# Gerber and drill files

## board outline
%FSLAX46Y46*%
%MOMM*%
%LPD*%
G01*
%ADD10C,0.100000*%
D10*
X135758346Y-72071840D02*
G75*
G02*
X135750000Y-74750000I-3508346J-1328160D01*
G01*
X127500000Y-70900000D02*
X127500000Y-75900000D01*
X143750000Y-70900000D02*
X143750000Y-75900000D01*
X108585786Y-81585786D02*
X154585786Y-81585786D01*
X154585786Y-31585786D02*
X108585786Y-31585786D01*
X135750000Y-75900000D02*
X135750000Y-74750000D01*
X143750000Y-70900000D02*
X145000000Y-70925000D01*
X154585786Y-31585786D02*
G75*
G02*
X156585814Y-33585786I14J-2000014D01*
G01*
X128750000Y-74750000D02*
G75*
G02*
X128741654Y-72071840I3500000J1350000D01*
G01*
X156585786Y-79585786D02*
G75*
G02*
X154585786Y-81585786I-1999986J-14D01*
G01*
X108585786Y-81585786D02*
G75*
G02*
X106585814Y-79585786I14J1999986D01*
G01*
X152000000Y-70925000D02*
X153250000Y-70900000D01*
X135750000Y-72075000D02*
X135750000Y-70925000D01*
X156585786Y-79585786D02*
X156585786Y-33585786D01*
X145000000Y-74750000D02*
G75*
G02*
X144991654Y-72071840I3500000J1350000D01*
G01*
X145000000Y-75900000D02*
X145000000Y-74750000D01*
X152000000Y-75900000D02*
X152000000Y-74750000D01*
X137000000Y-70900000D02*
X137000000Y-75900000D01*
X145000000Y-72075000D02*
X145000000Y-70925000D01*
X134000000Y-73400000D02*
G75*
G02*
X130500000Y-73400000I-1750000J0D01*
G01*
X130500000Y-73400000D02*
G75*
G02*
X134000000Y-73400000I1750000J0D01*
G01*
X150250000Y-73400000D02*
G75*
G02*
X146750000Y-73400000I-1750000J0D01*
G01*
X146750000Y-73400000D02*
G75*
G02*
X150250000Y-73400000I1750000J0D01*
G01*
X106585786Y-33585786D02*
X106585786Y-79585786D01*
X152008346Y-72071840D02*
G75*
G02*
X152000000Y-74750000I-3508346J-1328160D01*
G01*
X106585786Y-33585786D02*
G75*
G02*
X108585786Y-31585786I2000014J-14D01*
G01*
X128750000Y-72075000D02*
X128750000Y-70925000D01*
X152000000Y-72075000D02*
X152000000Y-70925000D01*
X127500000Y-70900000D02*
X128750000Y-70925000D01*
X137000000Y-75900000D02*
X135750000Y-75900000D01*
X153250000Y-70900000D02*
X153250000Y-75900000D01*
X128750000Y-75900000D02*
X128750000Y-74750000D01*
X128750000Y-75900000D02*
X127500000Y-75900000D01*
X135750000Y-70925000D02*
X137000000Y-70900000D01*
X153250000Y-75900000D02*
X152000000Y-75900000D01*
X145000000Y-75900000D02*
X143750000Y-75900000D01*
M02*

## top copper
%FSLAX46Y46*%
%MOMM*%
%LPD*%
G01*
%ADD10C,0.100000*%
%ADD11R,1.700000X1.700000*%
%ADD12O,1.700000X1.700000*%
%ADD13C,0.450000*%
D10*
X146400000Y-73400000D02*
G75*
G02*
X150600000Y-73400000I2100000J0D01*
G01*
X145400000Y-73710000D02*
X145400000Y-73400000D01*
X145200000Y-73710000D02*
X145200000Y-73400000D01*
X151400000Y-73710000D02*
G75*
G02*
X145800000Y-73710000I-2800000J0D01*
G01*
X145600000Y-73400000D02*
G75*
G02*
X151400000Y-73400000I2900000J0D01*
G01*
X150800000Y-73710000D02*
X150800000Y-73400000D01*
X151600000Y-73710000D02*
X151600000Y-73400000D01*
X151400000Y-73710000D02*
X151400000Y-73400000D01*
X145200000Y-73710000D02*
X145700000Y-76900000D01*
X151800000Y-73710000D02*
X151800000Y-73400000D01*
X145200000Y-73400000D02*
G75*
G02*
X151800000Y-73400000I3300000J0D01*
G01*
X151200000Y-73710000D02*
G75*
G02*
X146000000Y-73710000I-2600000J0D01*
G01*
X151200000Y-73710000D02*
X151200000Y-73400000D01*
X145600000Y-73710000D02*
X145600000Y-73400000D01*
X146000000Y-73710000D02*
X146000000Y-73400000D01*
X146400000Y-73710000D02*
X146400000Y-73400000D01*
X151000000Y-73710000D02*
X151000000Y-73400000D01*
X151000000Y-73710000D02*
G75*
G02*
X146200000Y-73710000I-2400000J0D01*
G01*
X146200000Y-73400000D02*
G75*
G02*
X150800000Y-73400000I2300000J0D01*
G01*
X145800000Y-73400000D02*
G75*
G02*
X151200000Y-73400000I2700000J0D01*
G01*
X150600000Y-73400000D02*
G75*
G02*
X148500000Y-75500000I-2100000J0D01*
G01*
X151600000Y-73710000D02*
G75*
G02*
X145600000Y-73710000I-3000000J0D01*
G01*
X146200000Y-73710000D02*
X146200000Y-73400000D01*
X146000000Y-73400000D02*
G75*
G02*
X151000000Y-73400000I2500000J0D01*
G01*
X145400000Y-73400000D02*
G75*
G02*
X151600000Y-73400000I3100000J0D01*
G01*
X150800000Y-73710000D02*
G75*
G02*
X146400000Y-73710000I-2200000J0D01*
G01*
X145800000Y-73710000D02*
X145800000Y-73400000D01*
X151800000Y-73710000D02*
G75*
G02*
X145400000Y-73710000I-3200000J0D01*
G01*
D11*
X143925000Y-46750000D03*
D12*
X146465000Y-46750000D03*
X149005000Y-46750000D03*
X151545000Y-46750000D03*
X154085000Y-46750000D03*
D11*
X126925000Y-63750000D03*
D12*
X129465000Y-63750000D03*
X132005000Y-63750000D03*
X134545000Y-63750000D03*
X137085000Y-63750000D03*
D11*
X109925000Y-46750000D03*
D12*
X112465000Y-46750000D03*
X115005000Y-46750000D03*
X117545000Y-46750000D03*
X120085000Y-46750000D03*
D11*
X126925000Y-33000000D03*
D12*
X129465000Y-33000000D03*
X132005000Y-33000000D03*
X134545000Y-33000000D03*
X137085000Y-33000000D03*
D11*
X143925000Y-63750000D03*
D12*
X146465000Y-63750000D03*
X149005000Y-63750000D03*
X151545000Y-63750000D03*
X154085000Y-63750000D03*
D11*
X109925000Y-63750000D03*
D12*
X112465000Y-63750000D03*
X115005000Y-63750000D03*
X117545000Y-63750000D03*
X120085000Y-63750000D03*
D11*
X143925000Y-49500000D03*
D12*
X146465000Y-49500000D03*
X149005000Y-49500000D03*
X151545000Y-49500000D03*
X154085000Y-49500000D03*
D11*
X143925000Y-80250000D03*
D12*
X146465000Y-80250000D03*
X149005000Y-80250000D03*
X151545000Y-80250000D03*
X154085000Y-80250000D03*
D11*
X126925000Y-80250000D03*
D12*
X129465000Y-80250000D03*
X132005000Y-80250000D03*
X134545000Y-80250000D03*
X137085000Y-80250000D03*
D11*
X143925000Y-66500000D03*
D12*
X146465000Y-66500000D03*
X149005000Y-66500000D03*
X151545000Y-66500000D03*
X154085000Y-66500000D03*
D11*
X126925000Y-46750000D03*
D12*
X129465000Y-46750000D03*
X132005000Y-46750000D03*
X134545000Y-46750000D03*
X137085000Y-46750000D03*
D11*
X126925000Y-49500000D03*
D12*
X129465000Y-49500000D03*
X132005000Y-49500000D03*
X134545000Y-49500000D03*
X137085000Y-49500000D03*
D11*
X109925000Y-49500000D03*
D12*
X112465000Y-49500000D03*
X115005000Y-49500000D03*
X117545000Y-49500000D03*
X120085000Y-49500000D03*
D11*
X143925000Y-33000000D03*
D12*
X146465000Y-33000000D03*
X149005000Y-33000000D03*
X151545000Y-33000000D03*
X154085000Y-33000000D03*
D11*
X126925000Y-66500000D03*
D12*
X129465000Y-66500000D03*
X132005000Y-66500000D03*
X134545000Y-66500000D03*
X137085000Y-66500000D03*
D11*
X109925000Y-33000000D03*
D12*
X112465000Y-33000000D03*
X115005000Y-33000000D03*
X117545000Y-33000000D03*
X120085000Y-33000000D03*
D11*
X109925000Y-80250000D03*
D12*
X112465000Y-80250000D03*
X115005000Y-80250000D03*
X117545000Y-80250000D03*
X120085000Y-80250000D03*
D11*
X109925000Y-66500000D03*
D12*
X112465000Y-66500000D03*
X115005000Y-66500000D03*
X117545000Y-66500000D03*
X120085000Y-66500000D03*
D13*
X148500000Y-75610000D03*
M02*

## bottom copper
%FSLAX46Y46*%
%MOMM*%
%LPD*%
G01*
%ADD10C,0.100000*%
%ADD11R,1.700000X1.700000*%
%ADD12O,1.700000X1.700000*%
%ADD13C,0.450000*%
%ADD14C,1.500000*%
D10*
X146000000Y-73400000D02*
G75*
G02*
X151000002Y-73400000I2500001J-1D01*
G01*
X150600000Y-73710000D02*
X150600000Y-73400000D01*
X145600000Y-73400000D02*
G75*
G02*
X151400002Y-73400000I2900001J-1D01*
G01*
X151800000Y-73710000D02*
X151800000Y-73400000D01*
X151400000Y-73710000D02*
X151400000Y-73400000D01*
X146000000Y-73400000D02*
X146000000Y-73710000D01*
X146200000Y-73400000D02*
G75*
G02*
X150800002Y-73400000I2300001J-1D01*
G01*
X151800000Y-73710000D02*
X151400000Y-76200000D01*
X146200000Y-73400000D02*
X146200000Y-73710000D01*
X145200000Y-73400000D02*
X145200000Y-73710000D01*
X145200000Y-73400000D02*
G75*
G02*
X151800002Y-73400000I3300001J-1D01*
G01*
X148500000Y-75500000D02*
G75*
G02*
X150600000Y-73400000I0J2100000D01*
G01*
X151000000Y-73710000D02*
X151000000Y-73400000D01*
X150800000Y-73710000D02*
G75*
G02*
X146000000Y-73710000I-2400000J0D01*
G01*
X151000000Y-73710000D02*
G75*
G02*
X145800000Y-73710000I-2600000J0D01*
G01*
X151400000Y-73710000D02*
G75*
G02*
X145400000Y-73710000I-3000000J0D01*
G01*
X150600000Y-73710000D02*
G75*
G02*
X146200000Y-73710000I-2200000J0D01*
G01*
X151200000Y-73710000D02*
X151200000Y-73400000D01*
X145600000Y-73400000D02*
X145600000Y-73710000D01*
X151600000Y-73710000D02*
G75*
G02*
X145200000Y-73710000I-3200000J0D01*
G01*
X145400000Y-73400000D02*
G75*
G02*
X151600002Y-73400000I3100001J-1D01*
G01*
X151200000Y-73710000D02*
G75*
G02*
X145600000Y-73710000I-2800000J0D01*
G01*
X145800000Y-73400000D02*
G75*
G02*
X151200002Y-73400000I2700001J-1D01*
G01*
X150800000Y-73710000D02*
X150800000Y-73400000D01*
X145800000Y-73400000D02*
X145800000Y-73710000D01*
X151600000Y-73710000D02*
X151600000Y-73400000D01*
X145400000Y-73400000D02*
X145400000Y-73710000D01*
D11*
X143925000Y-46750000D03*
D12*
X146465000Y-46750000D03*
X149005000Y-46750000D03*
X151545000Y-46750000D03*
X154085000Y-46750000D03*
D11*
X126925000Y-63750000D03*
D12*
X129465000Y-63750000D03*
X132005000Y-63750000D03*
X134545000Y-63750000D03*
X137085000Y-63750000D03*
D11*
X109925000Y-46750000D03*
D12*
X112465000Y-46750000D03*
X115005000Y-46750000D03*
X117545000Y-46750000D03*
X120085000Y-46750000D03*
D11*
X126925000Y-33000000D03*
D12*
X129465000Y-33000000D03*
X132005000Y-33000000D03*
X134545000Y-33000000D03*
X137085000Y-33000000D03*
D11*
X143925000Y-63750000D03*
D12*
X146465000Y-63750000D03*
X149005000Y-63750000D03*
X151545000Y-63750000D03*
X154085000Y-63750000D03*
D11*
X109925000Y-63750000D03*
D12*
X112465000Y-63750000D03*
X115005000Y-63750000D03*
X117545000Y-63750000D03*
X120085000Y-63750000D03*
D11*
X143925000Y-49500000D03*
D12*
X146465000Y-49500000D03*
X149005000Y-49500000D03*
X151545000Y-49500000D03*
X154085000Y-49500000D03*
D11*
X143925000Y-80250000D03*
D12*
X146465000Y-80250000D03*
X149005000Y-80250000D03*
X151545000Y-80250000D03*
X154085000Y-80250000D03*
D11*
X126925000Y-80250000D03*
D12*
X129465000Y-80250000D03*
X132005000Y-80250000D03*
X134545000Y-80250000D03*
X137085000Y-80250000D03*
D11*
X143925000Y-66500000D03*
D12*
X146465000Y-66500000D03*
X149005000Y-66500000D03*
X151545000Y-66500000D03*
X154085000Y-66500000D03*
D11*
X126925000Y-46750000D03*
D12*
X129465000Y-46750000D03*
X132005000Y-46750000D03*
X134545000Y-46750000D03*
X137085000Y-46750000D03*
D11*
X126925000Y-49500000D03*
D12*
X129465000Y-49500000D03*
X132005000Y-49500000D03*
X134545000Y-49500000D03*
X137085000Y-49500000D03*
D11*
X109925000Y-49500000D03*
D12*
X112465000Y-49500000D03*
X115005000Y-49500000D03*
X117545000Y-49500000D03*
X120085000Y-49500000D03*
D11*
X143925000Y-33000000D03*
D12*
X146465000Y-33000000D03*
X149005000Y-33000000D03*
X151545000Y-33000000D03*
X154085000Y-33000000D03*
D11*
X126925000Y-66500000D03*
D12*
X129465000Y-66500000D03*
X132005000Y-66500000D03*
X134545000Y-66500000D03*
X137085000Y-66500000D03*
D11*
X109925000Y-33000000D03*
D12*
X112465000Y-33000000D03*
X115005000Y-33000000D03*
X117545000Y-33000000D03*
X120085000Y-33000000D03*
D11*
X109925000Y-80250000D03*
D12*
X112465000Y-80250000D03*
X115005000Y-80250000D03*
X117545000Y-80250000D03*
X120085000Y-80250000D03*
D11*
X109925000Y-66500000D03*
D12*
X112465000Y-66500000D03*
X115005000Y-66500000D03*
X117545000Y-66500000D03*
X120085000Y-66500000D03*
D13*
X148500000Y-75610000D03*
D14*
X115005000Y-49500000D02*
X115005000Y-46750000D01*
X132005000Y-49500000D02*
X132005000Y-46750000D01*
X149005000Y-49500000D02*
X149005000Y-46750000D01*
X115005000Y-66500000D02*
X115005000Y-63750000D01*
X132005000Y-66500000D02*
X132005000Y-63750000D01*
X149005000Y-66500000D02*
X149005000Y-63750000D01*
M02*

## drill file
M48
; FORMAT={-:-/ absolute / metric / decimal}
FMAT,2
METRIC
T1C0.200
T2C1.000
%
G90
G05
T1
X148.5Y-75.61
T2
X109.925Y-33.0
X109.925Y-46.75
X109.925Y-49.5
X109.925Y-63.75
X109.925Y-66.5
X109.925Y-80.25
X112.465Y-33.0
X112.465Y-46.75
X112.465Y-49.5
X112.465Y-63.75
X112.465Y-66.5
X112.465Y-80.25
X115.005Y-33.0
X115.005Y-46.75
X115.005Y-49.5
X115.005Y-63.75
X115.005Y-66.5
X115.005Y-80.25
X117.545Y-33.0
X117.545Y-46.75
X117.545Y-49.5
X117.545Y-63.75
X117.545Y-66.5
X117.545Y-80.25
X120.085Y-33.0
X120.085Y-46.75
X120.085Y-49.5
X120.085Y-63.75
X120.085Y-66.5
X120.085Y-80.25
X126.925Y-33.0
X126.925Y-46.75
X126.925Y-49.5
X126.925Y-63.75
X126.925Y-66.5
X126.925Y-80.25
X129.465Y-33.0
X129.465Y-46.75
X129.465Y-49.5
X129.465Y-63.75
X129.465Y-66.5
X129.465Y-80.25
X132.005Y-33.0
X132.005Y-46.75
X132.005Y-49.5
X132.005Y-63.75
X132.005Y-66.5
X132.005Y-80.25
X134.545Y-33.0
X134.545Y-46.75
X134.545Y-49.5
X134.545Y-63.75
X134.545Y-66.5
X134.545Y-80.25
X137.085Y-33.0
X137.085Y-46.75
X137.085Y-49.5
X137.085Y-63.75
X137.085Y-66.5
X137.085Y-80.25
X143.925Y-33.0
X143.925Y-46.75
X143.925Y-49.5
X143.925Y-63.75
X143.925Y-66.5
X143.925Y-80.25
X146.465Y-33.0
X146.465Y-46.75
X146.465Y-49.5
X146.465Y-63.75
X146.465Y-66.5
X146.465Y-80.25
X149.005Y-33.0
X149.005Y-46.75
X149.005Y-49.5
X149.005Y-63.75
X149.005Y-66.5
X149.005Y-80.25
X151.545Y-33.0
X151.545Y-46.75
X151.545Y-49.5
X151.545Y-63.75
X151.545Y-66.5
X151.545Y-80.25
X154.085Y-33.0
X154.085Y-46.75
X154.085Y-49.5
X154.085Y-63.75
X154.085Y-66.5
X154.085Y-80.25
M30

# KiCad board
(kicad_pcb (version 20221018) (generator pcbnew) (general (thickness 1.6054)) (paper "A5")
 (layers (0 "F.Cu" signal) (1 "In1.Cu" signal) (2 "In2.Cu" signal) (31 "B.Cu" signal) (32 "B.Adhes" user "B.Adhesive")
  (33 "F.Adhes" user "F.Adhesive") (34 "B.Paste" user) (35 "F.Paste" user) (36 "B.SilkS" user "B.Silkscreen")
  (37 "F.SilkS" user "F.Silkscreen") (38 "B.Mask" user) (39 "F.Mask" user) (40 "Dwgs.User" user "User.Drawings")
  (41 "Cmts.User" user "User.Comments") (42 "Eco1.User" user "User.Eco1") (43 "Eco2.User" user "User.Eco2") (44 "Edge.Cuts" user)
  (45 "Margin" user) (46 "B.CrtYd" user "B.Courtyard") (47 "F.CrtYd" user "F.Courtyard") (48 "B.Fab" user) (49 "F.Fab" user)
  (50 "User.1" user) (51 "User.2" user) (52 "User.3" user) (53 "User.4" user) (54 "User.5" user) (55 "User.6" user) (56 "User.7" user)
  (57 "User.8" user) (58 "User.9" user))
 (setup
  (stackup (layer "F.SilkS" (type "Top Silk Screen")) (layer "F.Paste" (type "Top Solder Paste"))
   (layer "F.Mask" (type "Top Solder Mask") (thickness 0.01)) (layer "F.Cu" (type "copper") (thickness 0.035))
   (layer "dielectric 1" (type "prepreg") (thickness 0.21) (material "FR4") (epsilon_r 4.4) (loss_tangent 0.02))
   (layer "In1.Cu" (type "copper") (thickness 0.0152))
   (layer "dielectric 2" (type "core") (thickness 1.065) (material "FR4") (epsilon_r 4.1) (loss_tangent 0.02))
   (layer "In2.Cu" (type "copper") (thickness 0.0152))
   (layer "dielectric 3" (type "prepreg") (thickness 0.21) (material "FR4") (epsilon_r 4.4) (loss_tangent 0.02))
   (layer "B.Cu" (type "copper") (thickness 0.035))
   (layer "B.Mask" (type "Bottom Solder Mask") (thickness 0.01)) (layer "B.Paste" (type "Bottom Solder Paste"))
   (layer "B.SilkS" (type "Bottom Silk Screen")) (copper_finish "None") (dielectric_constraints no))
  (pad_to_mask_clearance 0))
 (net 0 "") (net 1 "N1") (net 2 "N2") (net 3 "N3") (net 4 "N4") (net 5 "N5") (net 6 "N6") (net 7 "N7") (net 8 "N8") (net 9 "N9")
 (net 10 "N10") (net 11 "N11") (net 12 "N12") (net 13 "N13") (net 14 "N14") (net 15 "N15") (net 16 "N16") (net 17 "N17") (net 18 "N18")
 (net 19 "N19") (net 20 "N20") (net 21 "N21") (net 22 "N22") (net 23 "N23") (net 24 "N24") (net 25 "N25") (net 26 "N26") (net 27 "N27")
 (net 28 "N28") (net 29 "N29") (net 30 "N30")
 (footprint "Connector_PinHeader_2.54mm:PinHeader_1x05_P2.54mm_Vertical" (layer "F.Cu") (at 143.925 46.75 90)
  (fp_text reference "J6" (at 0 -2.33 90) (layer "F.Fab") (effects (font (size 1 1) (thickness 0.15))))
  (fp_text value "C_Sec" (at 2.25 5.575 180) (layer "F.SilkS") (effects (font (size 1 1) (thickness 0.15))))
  (pad "1" thru_hole rect (at 0 0 90) (size 1.7 1.7) (drill 1) (layers "*.Cu" "*.Mask") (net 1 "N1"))
  (pad "2" thru_hole oval (at 0 2.54 90) (size 1.7 1.7) (drill 1) (layers "*.Cu" "*.Mask") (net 1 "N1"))
  (pad "3" thru_hole oval (at 0 5.08 90) (size 1.7 1.7) (drill 1) (layers "*.Cu" "*.Mask") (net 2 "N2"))
  (pad "4" thru_hole oval (at 0 7.62 90) (size 1.7 1.7) (drill 1) (layers "*.Cu" "*.Mask") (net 1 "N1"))
  (pad "5" thru_hole oval (at 0 10.16 90) (size 1.7 1.7) (drill 1) (layers "*.Cu" "*.Mask") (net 1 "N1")))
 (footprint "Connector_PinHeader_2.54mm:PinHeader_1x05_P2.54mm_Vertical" (layer "F.Cu") (at 126.925 63.75 90)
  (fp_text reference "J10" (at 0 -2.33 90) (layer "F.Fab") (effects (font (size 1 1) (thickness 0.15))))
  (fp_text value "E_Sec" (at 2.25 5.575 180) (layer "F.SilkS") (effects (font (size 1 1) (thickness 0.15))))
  (pad "1" thru_hole rect (at 0 0 90) (size 1.7 1.7) (drill 1) (layers "*.Cu" "*.Mask") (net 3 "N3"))
  (pad "2" thru_hole oval (at 0 2.54 90) (size 1.7 1.7) (drill 1) (layers "*.Cu" "*.Mask") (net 3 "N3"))
  (pad "3" thru_hole oval (at 0 5.08 90) (size 1.7 1.7) (drill 1) (layers "*.Cu" "*.Mask") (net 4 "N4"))
  (pad "4" thru_hole oval (at 0 7.62 90) (size 1.7 1.7) (drill 1) (layers "*.Cu" "*.Mask") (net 3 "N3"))
  (pad "5" thru_hole oval (at 0 10.16 90) (size 1.7 1.7) (drill 1) (layers "*.Cu" "*.Mask") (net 3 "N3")))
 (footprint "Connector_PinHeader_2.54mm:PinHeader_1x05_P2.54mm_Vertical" (layer "F.Cu") (at 109.925 46.75 90)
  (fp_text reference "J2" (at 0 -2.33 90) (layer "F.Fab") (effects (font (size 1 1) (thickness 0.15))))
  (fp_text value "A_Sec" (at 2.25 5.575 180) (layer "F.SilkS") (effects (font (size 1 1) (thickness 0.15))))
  (pad "1" thru_hole rect (at 0 0 90) (size 1.7 1.7) (drill 1) (layers "*.Cu" "*.Mask") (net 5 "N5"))
  (pad "2" thru_hole oval (at 0 2.54 90) (size 1.7 1.7) (drill 1) (layers "*.Cu" "*.Mask") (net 5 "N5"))
  (pad "3" thru_hole oval (at 0 5.08 90) (size 1.7 1.7) (drill 1) (layers "*.Cu" "*.Mask") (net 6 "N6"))
  (pad "4" thru_hole oval (at 0 7.62 90) (size 1.7 1.7) (drill 1) (layers "*.Cu" "*.Mask") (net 5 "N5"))
  (pad "5" thru_hole oval (at 0 10.16 90) (size 1.7 1.7) (drill 1) (layers "*.Cu" "*.Mask") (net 5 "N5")))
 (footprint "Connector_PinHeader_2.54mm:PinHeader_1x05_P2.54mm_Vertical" (layer "F.Cu") (at 126.925 33 90)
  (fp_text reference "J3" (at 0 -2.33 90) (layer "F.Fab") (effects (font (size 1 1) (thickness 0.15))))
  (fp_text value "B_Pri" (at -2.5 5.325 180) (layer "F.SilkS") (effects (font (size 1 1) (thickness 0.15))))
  (pad "1" thru_hole rect (at 0 0 90) (size 1.7 1.7) (drill 1) (layers "*.Cu" "*.Mask") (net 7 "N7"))
  (pad "2" thru_hole oval (at 0 2.54 90) (size 1.7 1.7) (drill 1) (layers "*.Cu" "*.Mask") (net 7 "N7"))
  (pad "3" thru_hole oval (at 0 5.08 90) (size 1.7 1.7) (drill 1) (layers "*.Cu" "*.Mask") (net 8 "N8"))
  (pad "4" thru_hole oval (at 0 7.62 90) (size 1.7 1.7) (drill 1) (layers "*.Cu" "*.Mask") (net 7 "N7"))
  (pad "5" thru_hole oval (at 0 10.16 90) (size 1.7 1.7) (drill 1) (layers "*.Cu" "*.Mask") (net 7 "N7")))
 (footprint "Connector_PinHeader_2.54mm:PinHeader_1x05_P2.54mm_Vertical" (layer "F.Cu") (at 143.925 63.75 90)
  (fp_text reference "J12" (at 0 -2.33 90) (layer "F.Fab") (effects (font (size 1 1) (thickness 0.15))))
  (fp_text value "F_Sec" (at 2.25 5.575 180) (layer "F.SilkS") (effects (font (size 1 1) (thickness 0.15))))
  (pad "1" thru_hole rect (at 0 0 90) (size 1.7 1.7) (drill 1) (layers "*.Cu" "*.Mask") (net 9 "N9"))
  (pad "2" thru_hole oval (at 0 2.54 90) (size 1.7 1.7) (drill 1) (layers "*.Cu" "*.Mask") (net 9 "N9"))
  (pad "3" thru_hole oval (at 0 5.08 90) (size 1.7 1.7) (drill 1) (layers "*.Cu" "*.Mask") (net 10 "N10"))
  (pad "4" thru_hole oval (at 0 7.62 90) (size 1.7 1.7) (drill 1) (layers "*.Cu" "*.Mask") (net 9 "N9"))
  (pad "5" thru_hole oval (at 0 10.16 90) (size 1.7 1.7) (drill 1) (layers "*.Cu" "*.Mask") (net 9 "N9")))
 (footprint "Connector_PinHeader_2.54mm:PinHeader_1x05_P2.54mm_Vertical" (layer "F.Cu") (at 109.925 63.75 90)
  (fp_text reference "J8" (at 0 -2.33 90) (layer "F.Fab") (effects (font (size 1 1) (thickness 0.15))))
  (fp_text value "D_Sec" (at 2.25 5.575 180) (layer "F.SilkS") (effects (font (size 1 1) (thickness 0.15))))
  (pad "1" thru_hole rect (at 0 0 90) (size 1.7 1.7) (drill 1) (layers "*.Cu" "*.Mask") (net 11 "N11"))
  (pad "2" thru_hole oval (at 0 2.54 90) (size 1.7 1.7) (drill 1) (layers "*.Cu" "*.Mask") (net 11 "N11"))
  (pad "3" thru_hole oval (at 0 5.08 90) (size 1.7 1.7) (drill 1) (layers "*.Cu" "*.Mask") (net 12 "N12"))
  (pad "4" thru_hole oval (at 0 7.62 90) (size 1.7 1.7) (drill 1) (layers "*.Cu" "*.Mask") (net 11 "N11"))
  (pad "5" thru_hole oval (at 0 10.16 90) (size 1.7 1.7) (drill 1) (layers "*.Cu" "*.Mask") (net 11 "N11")))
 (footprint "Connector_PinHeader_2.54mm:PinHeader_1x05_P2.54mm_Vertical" (layer "F.Cu") (at 143.925 49.5 90)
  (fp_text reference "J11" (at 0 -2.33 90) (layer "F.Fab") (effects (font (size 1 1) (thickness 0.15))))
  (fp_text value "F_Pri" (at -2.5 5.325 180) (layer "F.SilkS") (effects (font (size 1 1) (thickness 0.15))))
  (pad "1" thru_hole rect (at 0 0 90) (size 1.7 1.7) (drill 1) (layers "*.Cu" "*.Mask") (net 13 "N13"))
  (pad "2" thru_hole oval (at 0 2.54 90) (size 1.7 1.7) (drill 1) (layers "*.Cu" "*.Mask") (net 13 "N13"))
  (pad "3" thru_hole oval (at 0 5.08 90) (size 1.7 1.7) (drill 1) (layers "*.Cu" "*.Mask") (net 2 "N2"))
  (pad "4" thru_hole oval (at 0 7.62 90) (size 1.7 1.7) (drill 1) (layers "*.Cu" "*.Mask") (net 13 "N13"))
  (pad "5" thru_hole oval (at 0 10.16 90) (size 1.7 1.7) (drill 1) (layers "*.Cu" "*.Mask") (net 13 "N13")))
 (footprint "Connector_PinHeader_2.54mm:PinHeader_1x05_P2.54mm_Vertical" (layer "F.Cu") (at 143.925 80.25 90)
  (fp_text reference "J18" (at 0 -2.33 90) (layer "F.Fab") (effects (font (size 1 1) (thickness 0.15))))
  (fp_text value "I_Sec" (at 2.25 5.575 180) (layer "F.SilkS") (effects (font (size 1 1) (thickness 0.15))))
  (pad "1" thru_hole rect (at 0 0 90) (size 1.7 1.7) (drill 1) (layers "*.Cu" "*.Mask") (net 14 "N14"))
  (pad "2" thru_hole oval (at 0 2.54 90) (size 1.7 1.7) (drill 1) (layers "*.Cu" "*.Mask") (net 14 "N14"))
  (pad "3" thru_hole oval (at 0 5.08 90) (size 1.7 1.7) (drill 1) (layers "*.Cu" "*.Mask") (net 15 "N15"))
  (pad "4" thru_hole oval (at 0 7.62 90) (size 1.7 1.7) (drill 1) (layers "*.Cu" "*.Mask") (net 14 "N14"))
  (pad "5" thru_hole oval (at 0 10.16 90) (size 1.7 1.7) (drill 1) (layers "*.Cu" "*.Mask") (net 14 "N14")))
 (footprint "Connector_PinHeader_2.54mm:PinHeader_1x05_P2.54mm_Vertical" (layer "F.Cu") (at 126.925 80.25 90)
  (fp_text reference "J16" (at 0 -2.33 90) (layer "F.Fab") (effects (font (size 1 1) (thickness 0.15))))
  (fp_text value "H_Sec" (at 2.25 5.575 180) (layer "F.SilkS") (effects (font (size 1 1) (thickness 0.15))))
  (pad "1" thru_hole rect (at 0 0 90) (size 1.7 1.7) (drill 1) (layers "*.Cu" "*.Mask") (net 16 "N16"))
  (pad "2" thru_hole oval (at 0 2.54 90) (size 1.7 1.7) (drill 1) (layers "*.Cu" "*.Mask") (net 16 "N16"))
  (pad "3" thru_hole oval (at 0 5.08 90) (size 1.7 1.7) (drill 1) (layers "*.Cu" "*.Mask") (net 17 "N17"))
  (pad "4" thru_hole oval (at 0 7.62 90) (size 1.7 1.7) (drill 1) (layers "*.Cu" "*.Mask") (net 16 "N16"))
  (pad "5" thru_hole oval (at 0 10.16 90) (size 1.7 1.7) (drill 1) (layers "*.Cu" "*.Mask") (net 16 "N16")))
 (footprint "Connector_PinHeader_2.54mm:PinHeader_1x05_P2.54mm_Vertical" (layer "F.Cu") (at 143.925 66.5 90)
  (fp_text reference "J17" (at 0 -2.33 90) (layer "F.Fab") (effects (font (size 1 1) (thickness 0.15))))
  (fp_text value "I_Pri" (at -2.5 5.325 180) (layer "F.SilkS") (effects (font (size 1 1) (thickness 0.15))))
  (pad "1" thru_hole rect (at 0 0 90) (size 1.7 1.7) (drill 1) (layers "*.Cu" "*.Mask") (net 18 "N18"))
  (pad "2" thru_hole oval (at 0 2.54 90) (size 1.7 1.7) (drill 1) (layers "*.Cu" "*.Mask") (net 18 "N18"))
  (pad "3" thru_hole oval (at 0 5.08 90) (size 1.7 1.7) (drill 1) (layers "*.Cu" "*.Mask") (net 10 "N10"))
  (pad "4" thru_hole oval (at 0 7.62 90) (size 1.7 1.7) (drill 1) (layers "*.Cu" "*.Mask") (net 18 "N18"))
  (pad "5" thru_hole oval (at 0 10.16 90) (size 1.7 1.7) (drill 1) (layers "*.Cu" "*.Mask") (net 18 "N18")))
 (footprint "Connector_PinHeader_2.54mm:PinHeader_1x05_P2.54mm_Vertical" (layer "F.Cu") (at 126.925 46.75 90)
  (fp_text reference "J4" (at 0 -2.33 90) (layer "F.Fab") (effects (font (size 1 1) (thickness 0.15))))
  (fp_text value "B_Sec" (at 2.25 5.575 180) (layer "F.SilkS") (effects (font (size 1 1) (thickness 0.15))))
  (pad "1" thru_hole rect (at 0 0 90) (size 1.7 1.7) (drill 1) (layers "*.Cu" "*.Mask") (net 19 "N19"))
  (pad "2" thru_hole oval (at 0 2.54 90) (size 1.7 1.7) (drill 1) (layers "*.Cu" "*.Mask") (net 19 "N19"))
  (pad "3" thru_hole oval (at 0 5.08 90) (size 1.7 1.7) (drill 1) (layers "*.Cu" "*.Mask") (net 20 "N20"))
  (pad "4" thru_hole oval (at 0 7.62 90) (size 1.7 1.7) (drill 1) (layers "*.Cu" "*.Mask") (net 19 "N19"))
  (pad "5" thru_hole oval (at 0 10.16 90) (size 1.7 1.7) (drill 1) (layers "*.Cu" "*.Mask") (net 19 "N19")))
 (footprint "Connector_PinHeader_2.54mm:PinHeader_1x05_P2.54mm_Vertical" (layer "F.Cu") (at 126.925 49.5 90)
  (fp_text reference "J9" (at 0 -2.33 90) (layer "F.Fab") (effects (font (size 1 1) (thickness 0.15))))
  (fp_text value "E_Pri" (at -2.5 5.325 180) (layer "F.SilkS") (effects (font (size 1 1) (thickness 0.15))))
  (pad "1" thru_hole rect (at 0 0 90) (size 1.7 1.7) (drill 1) (layers "*.Cu" "*.Mask") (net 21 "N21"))
  (pad "2" thru_hole oval (at 0 2.54 90) (size 1.7 1.7) (drill 1) (layers "*.Cu" "*.Mask") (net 21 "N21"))
  (pad "3" thru_hole oval (at 0 5.08 90) (size 1.7 1.7) (drill 1) (layers "*.Cu" "*.Mask") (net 20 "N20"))
  (pad "4" thru_hole oval (at 0 7.62 90) (size 1.7 1.7) (drill 1) (layers "*.Cu" "*.Mask") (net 21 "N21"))
  (pad "5" thru_hole oval (at 0 10.16 90) (size 1.7 1.7) (drill 1) (layers "*.Cu" "*.Mask") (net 21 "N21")))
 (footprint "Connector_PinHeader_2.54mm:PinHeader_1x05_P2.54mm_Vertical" (layer "F.Cu") (at 109.925 49.5 90)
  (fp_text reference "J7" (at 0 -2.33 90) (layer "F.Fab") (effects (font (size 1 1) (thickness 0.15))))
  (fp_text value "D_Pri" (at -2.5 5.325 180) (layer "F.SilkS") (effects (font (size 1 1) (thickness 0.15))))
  (pad "1" thru_hole rect (at 0 0 90) (size 1.7 1.7) (drill 1) (layers "*.Cu" "*.Mask") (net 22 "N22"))
  (pad "2" thru_hole oval (at 0 2.54 90) (size 1.7 1.7) (drill 1) (layers "*.Cu" "*.Mask") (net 22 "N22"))
  (pad "3" thru_hole oval (at 0 5.08 90) (size 1.7 1.7) (drill 1) (layers "*.Cu" "*.Mask") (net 6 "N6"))
  (pad "4" thru_hole oval (at 0 7.62 90) (size 1.7 1.7) (drill 1) (layers "*.Cu" "*.Mask") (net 22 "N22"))
  (pad "5" thru_hole oval (at 0 10.16 90) (size 1.7 1.7) (drill 1) (layers "*.Cu" "*.Mask") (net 22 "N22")))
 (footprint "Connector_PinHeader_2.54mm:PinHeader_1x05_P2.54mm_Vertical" (layer "F.Cu") (at 143.925 33 90)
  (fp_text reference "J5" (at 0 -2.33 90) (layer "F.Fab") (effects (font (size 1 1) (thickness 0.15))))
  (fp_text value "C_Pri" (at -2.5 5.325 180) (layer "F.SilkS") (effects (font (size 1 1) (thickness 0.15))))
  (pad "1" thru_hole rect (at 0 0 90) (size 1.7 1.7) (drill 1) (layers "*.Cu" "*.Mask") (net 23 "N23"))
  (pad "2" thru_hole oval (at 0 2.54 90) (size 1.7 1.7) (drill 1) (layers "*.Cu" "*.Mask") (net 23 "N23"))
  (pad "3" thru_hole oval (at 0 5.08 90) (size 1.7 1.7) (drill 1) (layers "*.Cu" "*.Mask") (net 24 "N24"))
  (pad "4" thru_hole oval (at 0 7.62 90) (size 1.7 1.7) (drill 1) (layers "*.Cu" "*.Mask") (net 23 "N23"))
  (pad "5" thru_hole oval (at 0 10.16 90) (size 1.7 1.7) (drill 1) (layers "*.Cu" "*.Mask") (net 23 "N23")))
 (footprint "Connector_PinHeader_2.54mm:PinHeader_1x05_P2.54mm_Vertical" (layer "F.Cu") (at 126.925 66.5 90)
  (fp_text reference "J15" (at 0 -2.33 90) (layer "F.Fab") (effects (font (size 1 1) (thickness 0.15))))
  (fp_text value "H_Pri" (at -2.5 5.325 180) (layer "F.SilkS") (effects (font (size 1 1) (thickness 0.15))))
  (pad "1" thru_hole rect (at 0 0 90) (size 1.7 1.7) (drill 1) (layers "*.Cu" "*.Mask") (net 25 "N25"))
  (pad "2" thru_hole oval (at 0 2.54 90) (size 1.7 1.7) (drill 1) (layers "*.Cu" "*.Mask") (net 25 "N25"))
  (pad "3" thru_hole oval (at 0 5.08 90) (size 1.7 1.7) (drill 1) (layers "*.Cu" "*.Mask") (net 4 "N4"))
  (pad "4" thru_hole oval (at 0 7.62 90) (size 1.7 1.7) (drill 1) (layers "*.Cu" "*.Mask") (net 25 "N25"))
  (pad "5" thru_hole oval (at 0 10.16 90) (size 1.7 1.7) (drill 1) (layers "*.Cu" "*.Mask") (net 25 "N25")))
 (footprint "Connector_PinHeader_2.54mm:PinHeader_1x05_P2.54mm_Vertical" (layer "F.Cu") (at 109.925 33 90)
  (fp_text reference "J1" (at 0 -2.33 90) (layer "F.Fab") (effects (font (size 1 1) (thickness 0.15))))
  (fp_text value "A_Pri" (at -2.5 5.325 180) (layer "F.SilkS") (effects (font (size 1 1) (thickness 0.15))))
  (pad "1" thru_hole rect (at 0 0 90) (size 1.7 1.7) (drill 1) (layers "*.Cu" "*.Mask") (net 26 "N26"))
  (pad "2" thru_hole oval (at 0 2.54 90) (size 1.7 1.7) (drill 1) (layers "*.Cu" "*.Mask") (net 26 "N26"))
  (pad "3" thru_hole oval (at 0 5.08 90) (size 1.7 1.7) (drill 1) (layers "*.Cu" "*.Mask") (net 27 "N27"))
  (pad "4" thru_hole oval (at 0 7.62 90) (size 1.7 1.7) (drill 1) (layers "*.Cu" "*.Mask") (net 26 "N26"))
  (pad "5" thru_hole oval (at 0 10.16 90) (size 1.7 1.7) (drill 1) (layers "*.Cu" "*.Mask") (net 26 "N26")))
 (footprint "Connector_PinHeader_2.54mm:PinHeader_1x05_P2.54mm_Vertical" (layer "F.Cu") (at 109.925 80.25 90)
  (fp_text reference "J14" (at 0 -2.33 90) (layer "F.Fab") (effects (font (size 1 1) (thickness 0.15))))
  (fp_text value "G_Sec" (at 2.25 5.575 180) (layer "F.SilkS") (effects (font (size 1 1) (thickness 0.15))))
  (pad "1" thru_hole rect (at 0 0 90) (size 1.7 1.7) (drill 1) (layers "*.Cu" "*.Mask") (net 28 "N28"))
  (pad "2" thru_hole oval (at 0 2.54 90) (size 1.7 1.7) (drill 1) (layers "*.Cu" "*.Mask") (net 28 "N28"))
  (pad "3" thru_hole oval (at 0 5.08 90) (size 1.7 1.7) (drill 1) (layers "*.Cu" "*.Mask") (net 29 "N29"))
  (pad "4" thru_hole oval (at 0 7.62 90) (size 1.7 1.7) (drill 1) (layers "*.Cu" "*.Mask") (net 28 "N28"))
  (pad "5" thru_hole oval (at 0 10.16 90) (size 1.7 1.7) (drill 1) (layers "*.Cu" "*.Mask") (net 28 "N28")))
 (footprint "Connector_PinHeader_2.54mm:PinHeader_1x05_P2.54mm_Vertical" (layer "F.Cu") (at 109.925 66.5 90)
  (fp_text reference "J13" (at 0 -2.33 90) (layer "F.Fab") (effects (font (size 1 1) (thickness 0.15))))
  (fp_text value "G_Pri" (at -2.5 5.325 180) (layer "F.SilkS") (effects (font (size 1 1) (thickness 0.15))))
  (pad "1" thru_hole rect (at 0 0 90) (size 1.7 1.7) (drill 1) (layers "*.Cu" "*.Mask") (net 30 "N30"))
  (pad "2" thru_hole oval (at 0 2.54 90) (size 1.7 1.7) (drill 1) (layers "*.Cu" "*.Mask") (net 30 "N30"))
  (pad "3" thru_hole oval (at 0 5.08 90) (size 1.7 1.7) (drill 1) (layers "*.Cu" "*.Mask") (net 12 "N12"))
  (pad "4" thru_hole oval (at 0 7.62 90) (size 1.7 1.7) (drill 1) (layers "*.Cu" "*.Mask") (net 30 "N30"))
  (pad "5" thru_hole oval (at 0 10.16 90) (size 1.7 1.7) (drill 1) (layers "*.Cu" "*.Mask") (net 30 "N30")))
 (gr_arc (start 146.4 73.4) (mid 148.5 71.3) (end 150.6 73.4) (stroke (width 0.1) (type default)) (layer "F.Cu"))
 (gr_line (start 145.4 73.71) (end 145.4 73.4) (stroke (width 0.1) (type default)) (layer "F.Cu"))
 (gr_line (start 145.2 73.71) (end 145.2 73.4) (stroke (width 0.1) (type default)) (layer "F.Cu"))
 (gr_arc (start 151.4 73.71) (mid 148.6 76.51) (end 145.8 73.71) (stroke (width 0.1) (type default)) (layer "F.Cu"))
 (gr_arc (start 145.6 73.4) (mid 148.5 70.5) (end 151.4 73.4) (stroke (width 0.1) (type default)) (layer "F.Cu"))
 (gr_line (start 150.8 73.71) (end 150.8 73.4) (stroke (width 0.1) (type default)) (layer "F.Cu"))
 (gr_line (start 151.6 73.71) (end 151.6 73.4) (stroke (width 0.1) (type default)) (layer "F.Cu"))
 (gr_line (start 151.4 73.71) (end 151.4 73.4) (stroke (width 0.1) (type default)) (layer "F.Cu"))
 (gr_line (start 145.2 73.71) (end 145.7 76.9) (stroke (width 0.1) (type default)) (layer "F.Cu"))
 (gr_line (start 151.8 73.71) (end 151.8 73.4) (stroke (width 0.1) (type default)) (layer "F.Cu"))
 (gr_arc (start 145.2 73.4) (mid 148.5 70.1) (end 151.8 73.4) (stroke (width 0.1) (type default)) (layer "F.Cu"))
 (gr_arc (start 151.2 73.71) (mid 148.6 76.31) (end 146 73.71) (stroke (width 0.1) (type default)) (layer "F.Cu"))
 (gr_line (start 151.2 73.71) (end 151.2 73.4) (stroke (width 0.1) (type default)) (layer "F.Cu"))
 (gr_line (start 145.6 73.71) (end 145.6 73.4) (stroke (width 0.1) (type default)) (layer "F.Cu"))
 (gr_line (start 146 73.71) (end 146 73.4) (stroke (width 0.1) (type default)) (layer "F.Cu"))
 (gr_line (start 146.4 73.71) (end 146.4 73.4) (stroke (width 0.1) (type default)) (layer "F.Cu"))
 (gr_line (start 151 73.71) (end 151 73.4) (stroke (width 0.1) (type default)) (layer "F.Cu"))
 (gr_arc (start 151 73.71) (mid 148.6 76.11) (end 146.2 73.71) (stroke (width 0.1) (type default)) (layer "F.Cu"))
 (gr_arc (start 146.2 73.4) (mid 148.5 71.1) (end 150.8 73.4) (stroke (width 0.1) (type default)) (layer "F.Cu"))
 (gr_arc (start 145.8 73.4) (mid 148.5 70.7) (end 151.2 73.4) (stroke (width 0.1) (type default)) (layer "F.Cu"))
 (gr_arc (start 150.6 73.4) (mid 149.984924 74.884924) (end 148.5 75.5) (stroke (width 0.1) (type default)) (layer "F.Cu"))
 (gr_arc (start 151.6 73.71) (mid 148.6 76.71) (end 145.6 73.71) (stroke (width 0.1) (type default)) (layer "F.Cu"))
 (gr_line (start 146.2 73.71) (end 146.2 73.4) (stroke (width 0.1) (type default)) (layer "F.Cu"))
 (gr_arc (start 146 73.4) (mid 148.5 70.9) (end 151 73.4) (stroke (width 0.1) (type default)) (layer "F.Cu"))
 (gr_arc (start 145.4 73.4) (mid 148.5 70.3) (end 151.6 73.4) (stroke (width 0.1) (type default)) (layer "F.Cu"))
 (gr_arc (start 150.8 73.71) (mid 148.6 75.91) (end 146.4 73.71) (stroke (width 0.1) (type default)) (layer "F.Cu"))
 (gr_line (start 145.8 73.71) (end 145.8 73.4) (stroke (width 0.1) (type default)) (layer "F.Cu"))
 (gr_arc (start 151.8 73.71) (mid 148.6 76.91) (end 145.4 73.71) (stroke (width 0.1) (type default)) (layer "F.Cu"))
 (gr_arc (start 146 73.4) (mid 148.500001 70.9) (end 151.000002 73.4) (stroke (width 0.1) (type default)) (layer "B.Cu"))
 (gr_line (start 150.6 73.71) (end 150.6 73.4) (stroke (width 0.1) (type default)) (layer "B.Cu"))
 (gr_arc (start 145.6 73.4) (mid 148.500001 70.5) (end 151.400002 73.4) (stroke (width 0.1) (type default)) (layer "B.Cu"))
 (gr_line (start 151.8 73.71) (end 151.8 73.4) (stroke (width 0.1) (type default)) (layer "B.Cu"))
 (gr_line (start 151.4 73.71) (end 151.4 73.4) (stroke (width 0.1) (type default)) (layer "B.Cu"))
 (gr_line (start 146 73.4) (end 146 73.71) (stroke (width 0.1) (type default)) (layer "B.Cu"))
 (gr_arc (start 146.2 73.4) (mid 148.500001 71.1) (end 150.800002 73.4) (stroke (width 0.1) (type default)) (layer "B.Cu"))
 (gr_line (start 151.8 73.71) (end 151.4 76.2) (stroke (width 0.1) (type default)) (layer "B.Cu"))
 (gr_line (start 146.2 73.4) (end 146.2 73.71) (stroke (width 0.1) (type default)) (layer "B.Cu"))
 (gr_line (start 145.2 73.4) (end 145.2 73.71) (stroke (width 0.1) (type default)) (layer "B.Cu"))
 (gr_arc (start 145.2 73.4) (mid 148.500001 70.1) (end 151.800002 73.4) (stroke (width 0.1) (type default)) (layer "B.Cu"))
 (gr_arc (start 148.5 75.5) (mid 147.015077 71.915077) (end 150.6 73.4) (stroke (width 0.1) (type default)) (layer "B.Cu"))
 (gr_line (start 151 73.71) (end 151 73.4) (stroke (width 0.1) (type default)) (layer "B.Cu"))
 (gr_arc (start 150.8 73.71) (mid 148.4 76.11) (end 146 73.71) (stroke (width 0.1) (type default)) (layer "B.Cu"))
 (gr_arc (start 151 73.71) (mid 148.4 76.31) (end 145.8 73.71) (stroke (width 0.1) (type default)) (layer "B.Cu"))
 (gr_arc (start 151.4 73.71) (mid 148.4 76.71) (end 145.4 73.71) (stroke (width 0.1) (type default)) (layer "B.Cu"))
 (gr_arc (start 150.6 73.71) (mid 148.4 75.91) (end 146.2 73.71) (stroke (width 0.1) (type default)) (layer "B.Cu"))
 (gr_line (start 151.2 73.71) (end 151.2 73.4) (stroke (width 0.1) (type default)) (layer "B.Cu"))
 (gr_line (start 145.6 73.4) (end 145.6 73.71) (stroke (width 0.1) (type default)) (layer "B.Cu"))
 (gr_arc (start 151.6 73.71) (mid 148.4 76.91) (end 145.2 73.71) (stroke (width 0.1) (type default)) (layer "B.Cu"))
 (gr_arc (start 145.4 73.4) (mid 148.500001 70.3) (end 151.600002 73.4) (stroke (width 0.1) (type default)) (layer "B.Cu"))
 (gr_arc (start 151.2 73.71) (mid 148.4 76.51) (end 145.6 73.71) (stroke (width 0.1) (type default)) (layer "B.Cu"))
 (gr_arc (start 145.8 73.4) (mid 148.500001 70.7) (end 151.200002 73.4) (stroke (width 0.1) (type default)) (layer "B.Cu"))
 (gr_line (start 150.8 73.71) (end 150.8 73.4) (stroke (width 0.1) (type default)) (layer "B.Cu"))
 (gr_line (start 145.8 73.4) (end 145.8 73.71) (stroke (width 0.1) (type default)) (layer "B.Cu"))
 (gr_line (start 151.6 73.71) (end 151.6 73.4) (stroke (width 0.1) (type default)) (layer "B.Cu"))
 (gr_line (start 145.4 73.4) (end 145.4 73.71) (stroke (width 0.1) (type default)) (layer "B.Cu"))
 (gr_arc (start 135.758346 72.07184) (mid 136.001315 73.41169) (end 135.75 74.75) (stroke (width 0.1) (type default)) (layer "Edge.Cuts"))
 (gr_line (start 127.5 70.9) (end 127.5 75.9) (stroke (width 0.1) (type default)) (layer "Edge.Cuts"))
 (gr_line (start 143.75 70.9) (end 143.75 75.9) (stroke (width 0.1) (type default)) (layer "Edge.Cuts"))
 (gr_line (start 108.585786 81.585786) (end 154.585786 81.585786) (stroke (width 0.1) (type default)) (layer "Edge.Cuts"))
 (gr_line (start 154.585786 31.585786) (end 108.585786 31.585786) (stroke (width 0.1) (type default)) (layer "Edge.Cuts"))
 (gr_line (start 135.75 75.9) (end 135.75 74.75) (stroke (width 0.1) (type default)) (layer "Edge.Cuts"))
 (gr_line (start 143.75 70.9) (end 145 70.925) (stroke (width 0.1) (type default)) (layer "Edge.Cuts"))
 (gr_arc (start 154.585786 31.585786) (mid 156 32.171572) (end 156.585786 33.585786) (stroke (width 0.1) (type default)) (layer "Edge.Cuts"))
 (gr_arc (start 128.75 74.75) (mid 128.498685 73.41169) (end 128.741654 72.07184) (stroke (width 0.1) (type default)) (layer "Edge.Cuts"))
 (gr_arc (start 156.585786 79.585786) (mid 156 81) (end 154.585786 81.585786) (stroke (width 0.1) (type default)) (layer "Edge.Cuts"))
 (gr_arc (start 108.585786 81.585786) (mid 107.171572 81) (end 106.585786 79.585786) (stroke (width 0.1) (type default)) (layer "Edge.Cuts"))
 (gr_line (start 152 70.925) (end 153.25 70.9) (stroke (width 0.1) (type default)) (layer "Edge.Cuts"))
 (gr_line (start 135.75 72.075) (end 135.75 70.925) (stroke (width 0.1) (type default)) (layer "Edge.Cuts"))
 (gr_line (start 156.585786 79.585786) (end 156.585786 33.585786) (stroke (width 0.1) (type default)) (layer "Edge.Cuts"))
 (gr_arc (start 145 74.75) (mid 144.748685 73.41169) (end 144.991654 72.07184) (stroke (width 0.1) (type default)) (layer "Edge.Cuts"))
 (gr_line (start 145 75.9) (end 145 74.75) (stroke (width 0.1) (type default)) (layer "Edge.Cuts"))
 (gr_line (start 152 75.9) (end 152 74.75) (stroke (width 0.1) (type default)) (layer "Edge.Cuts"))
 (gr_line (start 137 70.9) (end 137 75.9) (stroke (width 0.1) (type default)) (layer "Edge.Cuts"))
 (gr_line (start 145 72.075) (end 145 70.925) (stroke (width 0.1) (type default)) (layer "Edge.Cuts"))
 (gr_circle (center 132.25 73.4) (end 134 73.4) (stroke (width 0.1) (type default)) (fill none) (layer "Edge.Cuts"))
 (gr_circle (center 148.5 73.4) (end 150.25 73.4) (stroke (width 0.1) (type default)) (fill none) (layer "Edge.Cuts"))
 (gr_line (start 106.585786 33.585786) (end 106.585786 79.585786) (stroke (width 0.1) (type default)) (layer "Edge.Cuts"))
 (gr_arc (start 152.008346 72.07184) (mid 152.251315 73.41169) (end 152 74.75) (stroke (width 0.1) (type default)) (layer "Edge.Cuts"))
 (gr_arc (start 106.585786 33.585786) (mid 107.171572 32.171572) (end 108.585786 31.585786) (stroke (width 0.1) (type default))
  (layer "Edge.Cuts"))
 (gr_line (start 128.75 72.075) (end 128.75 70.925) (stroke (width 0.1) (type default)) (layer "Edge.Cuts"))
 (gr_line (start 152 72.075) (end 152 70.925) (stroke (width 0.1) (type default)) (layer "Edge.Cuts"))
 (gr_line (start 127.5 70.9) (end 128.75 70.925) (stroke (width 0.1) (type default)) (layer "Edge.Cuts"))
 (gr_line (start 137 75.9) (end 135.75 75.9) (stroke (width 0.1) (type default)) (layer "Edge.Cuts"))
 (gr_line (start 153.25 70.9) (end 153.25 75.9) (stroke (width 0.1) (type default)) (layer "Edge.Cuts"))
 (gr_line (start 128.75 75.9) (end 128.75 74.75) (stroke (width 0.1) (type default)) (layer "Edge.Cuts"))
 (gr_line (start 128.75 75.9) (end 127.5 75.9) (stroke (width 0.1) (type default)) (layer "Edge.Cuts"))
 (gr_line (start 135.75 70.925) (end 137 70.9) (stroke (width 0.1) (type default)) (layer "Edge.Cuts"))
 (gr_line (start 153.25 75.9) (end 152 75.9) (stroke (width 0.1) (type default)) (layer "Edge.Cuts"))
 (gr_line (start 145 75.9) (end 143.75 75.9) (stroke (width 0.1) (type default)) (layer "Edge.Cuts"))
 (via (at 148.5 75.61) (size 0.45) (drill 0.2) (layers "F.Cu" "B.Cu") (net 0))
 (segment (start 115.005 49.5) (end 115.005 46.75) (width 1.5) (layer "B.Cu") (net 6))
 (segment (start 132.005 49.5) (end 132.005 46.75) (width 1.5) (layer "B.Cu") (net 20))
 (segment (start 149.005 49.5) (end 149.005 46.75) (width 1.5) (layer "B.Cu") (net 2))
 (segment (start 115.005 66.5) (end 115.005 63.75) (width 1.5) (layer "B.Cu") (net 12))
 (segment (start 132.005 66.5) (end 132.005 63.75) (width 1.5) (layer "B.Cu") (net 4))
 (segment (start 149.005 66.5) (end 149.005 63.75) (width 1.5) (layer "B.Cu") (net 10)))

